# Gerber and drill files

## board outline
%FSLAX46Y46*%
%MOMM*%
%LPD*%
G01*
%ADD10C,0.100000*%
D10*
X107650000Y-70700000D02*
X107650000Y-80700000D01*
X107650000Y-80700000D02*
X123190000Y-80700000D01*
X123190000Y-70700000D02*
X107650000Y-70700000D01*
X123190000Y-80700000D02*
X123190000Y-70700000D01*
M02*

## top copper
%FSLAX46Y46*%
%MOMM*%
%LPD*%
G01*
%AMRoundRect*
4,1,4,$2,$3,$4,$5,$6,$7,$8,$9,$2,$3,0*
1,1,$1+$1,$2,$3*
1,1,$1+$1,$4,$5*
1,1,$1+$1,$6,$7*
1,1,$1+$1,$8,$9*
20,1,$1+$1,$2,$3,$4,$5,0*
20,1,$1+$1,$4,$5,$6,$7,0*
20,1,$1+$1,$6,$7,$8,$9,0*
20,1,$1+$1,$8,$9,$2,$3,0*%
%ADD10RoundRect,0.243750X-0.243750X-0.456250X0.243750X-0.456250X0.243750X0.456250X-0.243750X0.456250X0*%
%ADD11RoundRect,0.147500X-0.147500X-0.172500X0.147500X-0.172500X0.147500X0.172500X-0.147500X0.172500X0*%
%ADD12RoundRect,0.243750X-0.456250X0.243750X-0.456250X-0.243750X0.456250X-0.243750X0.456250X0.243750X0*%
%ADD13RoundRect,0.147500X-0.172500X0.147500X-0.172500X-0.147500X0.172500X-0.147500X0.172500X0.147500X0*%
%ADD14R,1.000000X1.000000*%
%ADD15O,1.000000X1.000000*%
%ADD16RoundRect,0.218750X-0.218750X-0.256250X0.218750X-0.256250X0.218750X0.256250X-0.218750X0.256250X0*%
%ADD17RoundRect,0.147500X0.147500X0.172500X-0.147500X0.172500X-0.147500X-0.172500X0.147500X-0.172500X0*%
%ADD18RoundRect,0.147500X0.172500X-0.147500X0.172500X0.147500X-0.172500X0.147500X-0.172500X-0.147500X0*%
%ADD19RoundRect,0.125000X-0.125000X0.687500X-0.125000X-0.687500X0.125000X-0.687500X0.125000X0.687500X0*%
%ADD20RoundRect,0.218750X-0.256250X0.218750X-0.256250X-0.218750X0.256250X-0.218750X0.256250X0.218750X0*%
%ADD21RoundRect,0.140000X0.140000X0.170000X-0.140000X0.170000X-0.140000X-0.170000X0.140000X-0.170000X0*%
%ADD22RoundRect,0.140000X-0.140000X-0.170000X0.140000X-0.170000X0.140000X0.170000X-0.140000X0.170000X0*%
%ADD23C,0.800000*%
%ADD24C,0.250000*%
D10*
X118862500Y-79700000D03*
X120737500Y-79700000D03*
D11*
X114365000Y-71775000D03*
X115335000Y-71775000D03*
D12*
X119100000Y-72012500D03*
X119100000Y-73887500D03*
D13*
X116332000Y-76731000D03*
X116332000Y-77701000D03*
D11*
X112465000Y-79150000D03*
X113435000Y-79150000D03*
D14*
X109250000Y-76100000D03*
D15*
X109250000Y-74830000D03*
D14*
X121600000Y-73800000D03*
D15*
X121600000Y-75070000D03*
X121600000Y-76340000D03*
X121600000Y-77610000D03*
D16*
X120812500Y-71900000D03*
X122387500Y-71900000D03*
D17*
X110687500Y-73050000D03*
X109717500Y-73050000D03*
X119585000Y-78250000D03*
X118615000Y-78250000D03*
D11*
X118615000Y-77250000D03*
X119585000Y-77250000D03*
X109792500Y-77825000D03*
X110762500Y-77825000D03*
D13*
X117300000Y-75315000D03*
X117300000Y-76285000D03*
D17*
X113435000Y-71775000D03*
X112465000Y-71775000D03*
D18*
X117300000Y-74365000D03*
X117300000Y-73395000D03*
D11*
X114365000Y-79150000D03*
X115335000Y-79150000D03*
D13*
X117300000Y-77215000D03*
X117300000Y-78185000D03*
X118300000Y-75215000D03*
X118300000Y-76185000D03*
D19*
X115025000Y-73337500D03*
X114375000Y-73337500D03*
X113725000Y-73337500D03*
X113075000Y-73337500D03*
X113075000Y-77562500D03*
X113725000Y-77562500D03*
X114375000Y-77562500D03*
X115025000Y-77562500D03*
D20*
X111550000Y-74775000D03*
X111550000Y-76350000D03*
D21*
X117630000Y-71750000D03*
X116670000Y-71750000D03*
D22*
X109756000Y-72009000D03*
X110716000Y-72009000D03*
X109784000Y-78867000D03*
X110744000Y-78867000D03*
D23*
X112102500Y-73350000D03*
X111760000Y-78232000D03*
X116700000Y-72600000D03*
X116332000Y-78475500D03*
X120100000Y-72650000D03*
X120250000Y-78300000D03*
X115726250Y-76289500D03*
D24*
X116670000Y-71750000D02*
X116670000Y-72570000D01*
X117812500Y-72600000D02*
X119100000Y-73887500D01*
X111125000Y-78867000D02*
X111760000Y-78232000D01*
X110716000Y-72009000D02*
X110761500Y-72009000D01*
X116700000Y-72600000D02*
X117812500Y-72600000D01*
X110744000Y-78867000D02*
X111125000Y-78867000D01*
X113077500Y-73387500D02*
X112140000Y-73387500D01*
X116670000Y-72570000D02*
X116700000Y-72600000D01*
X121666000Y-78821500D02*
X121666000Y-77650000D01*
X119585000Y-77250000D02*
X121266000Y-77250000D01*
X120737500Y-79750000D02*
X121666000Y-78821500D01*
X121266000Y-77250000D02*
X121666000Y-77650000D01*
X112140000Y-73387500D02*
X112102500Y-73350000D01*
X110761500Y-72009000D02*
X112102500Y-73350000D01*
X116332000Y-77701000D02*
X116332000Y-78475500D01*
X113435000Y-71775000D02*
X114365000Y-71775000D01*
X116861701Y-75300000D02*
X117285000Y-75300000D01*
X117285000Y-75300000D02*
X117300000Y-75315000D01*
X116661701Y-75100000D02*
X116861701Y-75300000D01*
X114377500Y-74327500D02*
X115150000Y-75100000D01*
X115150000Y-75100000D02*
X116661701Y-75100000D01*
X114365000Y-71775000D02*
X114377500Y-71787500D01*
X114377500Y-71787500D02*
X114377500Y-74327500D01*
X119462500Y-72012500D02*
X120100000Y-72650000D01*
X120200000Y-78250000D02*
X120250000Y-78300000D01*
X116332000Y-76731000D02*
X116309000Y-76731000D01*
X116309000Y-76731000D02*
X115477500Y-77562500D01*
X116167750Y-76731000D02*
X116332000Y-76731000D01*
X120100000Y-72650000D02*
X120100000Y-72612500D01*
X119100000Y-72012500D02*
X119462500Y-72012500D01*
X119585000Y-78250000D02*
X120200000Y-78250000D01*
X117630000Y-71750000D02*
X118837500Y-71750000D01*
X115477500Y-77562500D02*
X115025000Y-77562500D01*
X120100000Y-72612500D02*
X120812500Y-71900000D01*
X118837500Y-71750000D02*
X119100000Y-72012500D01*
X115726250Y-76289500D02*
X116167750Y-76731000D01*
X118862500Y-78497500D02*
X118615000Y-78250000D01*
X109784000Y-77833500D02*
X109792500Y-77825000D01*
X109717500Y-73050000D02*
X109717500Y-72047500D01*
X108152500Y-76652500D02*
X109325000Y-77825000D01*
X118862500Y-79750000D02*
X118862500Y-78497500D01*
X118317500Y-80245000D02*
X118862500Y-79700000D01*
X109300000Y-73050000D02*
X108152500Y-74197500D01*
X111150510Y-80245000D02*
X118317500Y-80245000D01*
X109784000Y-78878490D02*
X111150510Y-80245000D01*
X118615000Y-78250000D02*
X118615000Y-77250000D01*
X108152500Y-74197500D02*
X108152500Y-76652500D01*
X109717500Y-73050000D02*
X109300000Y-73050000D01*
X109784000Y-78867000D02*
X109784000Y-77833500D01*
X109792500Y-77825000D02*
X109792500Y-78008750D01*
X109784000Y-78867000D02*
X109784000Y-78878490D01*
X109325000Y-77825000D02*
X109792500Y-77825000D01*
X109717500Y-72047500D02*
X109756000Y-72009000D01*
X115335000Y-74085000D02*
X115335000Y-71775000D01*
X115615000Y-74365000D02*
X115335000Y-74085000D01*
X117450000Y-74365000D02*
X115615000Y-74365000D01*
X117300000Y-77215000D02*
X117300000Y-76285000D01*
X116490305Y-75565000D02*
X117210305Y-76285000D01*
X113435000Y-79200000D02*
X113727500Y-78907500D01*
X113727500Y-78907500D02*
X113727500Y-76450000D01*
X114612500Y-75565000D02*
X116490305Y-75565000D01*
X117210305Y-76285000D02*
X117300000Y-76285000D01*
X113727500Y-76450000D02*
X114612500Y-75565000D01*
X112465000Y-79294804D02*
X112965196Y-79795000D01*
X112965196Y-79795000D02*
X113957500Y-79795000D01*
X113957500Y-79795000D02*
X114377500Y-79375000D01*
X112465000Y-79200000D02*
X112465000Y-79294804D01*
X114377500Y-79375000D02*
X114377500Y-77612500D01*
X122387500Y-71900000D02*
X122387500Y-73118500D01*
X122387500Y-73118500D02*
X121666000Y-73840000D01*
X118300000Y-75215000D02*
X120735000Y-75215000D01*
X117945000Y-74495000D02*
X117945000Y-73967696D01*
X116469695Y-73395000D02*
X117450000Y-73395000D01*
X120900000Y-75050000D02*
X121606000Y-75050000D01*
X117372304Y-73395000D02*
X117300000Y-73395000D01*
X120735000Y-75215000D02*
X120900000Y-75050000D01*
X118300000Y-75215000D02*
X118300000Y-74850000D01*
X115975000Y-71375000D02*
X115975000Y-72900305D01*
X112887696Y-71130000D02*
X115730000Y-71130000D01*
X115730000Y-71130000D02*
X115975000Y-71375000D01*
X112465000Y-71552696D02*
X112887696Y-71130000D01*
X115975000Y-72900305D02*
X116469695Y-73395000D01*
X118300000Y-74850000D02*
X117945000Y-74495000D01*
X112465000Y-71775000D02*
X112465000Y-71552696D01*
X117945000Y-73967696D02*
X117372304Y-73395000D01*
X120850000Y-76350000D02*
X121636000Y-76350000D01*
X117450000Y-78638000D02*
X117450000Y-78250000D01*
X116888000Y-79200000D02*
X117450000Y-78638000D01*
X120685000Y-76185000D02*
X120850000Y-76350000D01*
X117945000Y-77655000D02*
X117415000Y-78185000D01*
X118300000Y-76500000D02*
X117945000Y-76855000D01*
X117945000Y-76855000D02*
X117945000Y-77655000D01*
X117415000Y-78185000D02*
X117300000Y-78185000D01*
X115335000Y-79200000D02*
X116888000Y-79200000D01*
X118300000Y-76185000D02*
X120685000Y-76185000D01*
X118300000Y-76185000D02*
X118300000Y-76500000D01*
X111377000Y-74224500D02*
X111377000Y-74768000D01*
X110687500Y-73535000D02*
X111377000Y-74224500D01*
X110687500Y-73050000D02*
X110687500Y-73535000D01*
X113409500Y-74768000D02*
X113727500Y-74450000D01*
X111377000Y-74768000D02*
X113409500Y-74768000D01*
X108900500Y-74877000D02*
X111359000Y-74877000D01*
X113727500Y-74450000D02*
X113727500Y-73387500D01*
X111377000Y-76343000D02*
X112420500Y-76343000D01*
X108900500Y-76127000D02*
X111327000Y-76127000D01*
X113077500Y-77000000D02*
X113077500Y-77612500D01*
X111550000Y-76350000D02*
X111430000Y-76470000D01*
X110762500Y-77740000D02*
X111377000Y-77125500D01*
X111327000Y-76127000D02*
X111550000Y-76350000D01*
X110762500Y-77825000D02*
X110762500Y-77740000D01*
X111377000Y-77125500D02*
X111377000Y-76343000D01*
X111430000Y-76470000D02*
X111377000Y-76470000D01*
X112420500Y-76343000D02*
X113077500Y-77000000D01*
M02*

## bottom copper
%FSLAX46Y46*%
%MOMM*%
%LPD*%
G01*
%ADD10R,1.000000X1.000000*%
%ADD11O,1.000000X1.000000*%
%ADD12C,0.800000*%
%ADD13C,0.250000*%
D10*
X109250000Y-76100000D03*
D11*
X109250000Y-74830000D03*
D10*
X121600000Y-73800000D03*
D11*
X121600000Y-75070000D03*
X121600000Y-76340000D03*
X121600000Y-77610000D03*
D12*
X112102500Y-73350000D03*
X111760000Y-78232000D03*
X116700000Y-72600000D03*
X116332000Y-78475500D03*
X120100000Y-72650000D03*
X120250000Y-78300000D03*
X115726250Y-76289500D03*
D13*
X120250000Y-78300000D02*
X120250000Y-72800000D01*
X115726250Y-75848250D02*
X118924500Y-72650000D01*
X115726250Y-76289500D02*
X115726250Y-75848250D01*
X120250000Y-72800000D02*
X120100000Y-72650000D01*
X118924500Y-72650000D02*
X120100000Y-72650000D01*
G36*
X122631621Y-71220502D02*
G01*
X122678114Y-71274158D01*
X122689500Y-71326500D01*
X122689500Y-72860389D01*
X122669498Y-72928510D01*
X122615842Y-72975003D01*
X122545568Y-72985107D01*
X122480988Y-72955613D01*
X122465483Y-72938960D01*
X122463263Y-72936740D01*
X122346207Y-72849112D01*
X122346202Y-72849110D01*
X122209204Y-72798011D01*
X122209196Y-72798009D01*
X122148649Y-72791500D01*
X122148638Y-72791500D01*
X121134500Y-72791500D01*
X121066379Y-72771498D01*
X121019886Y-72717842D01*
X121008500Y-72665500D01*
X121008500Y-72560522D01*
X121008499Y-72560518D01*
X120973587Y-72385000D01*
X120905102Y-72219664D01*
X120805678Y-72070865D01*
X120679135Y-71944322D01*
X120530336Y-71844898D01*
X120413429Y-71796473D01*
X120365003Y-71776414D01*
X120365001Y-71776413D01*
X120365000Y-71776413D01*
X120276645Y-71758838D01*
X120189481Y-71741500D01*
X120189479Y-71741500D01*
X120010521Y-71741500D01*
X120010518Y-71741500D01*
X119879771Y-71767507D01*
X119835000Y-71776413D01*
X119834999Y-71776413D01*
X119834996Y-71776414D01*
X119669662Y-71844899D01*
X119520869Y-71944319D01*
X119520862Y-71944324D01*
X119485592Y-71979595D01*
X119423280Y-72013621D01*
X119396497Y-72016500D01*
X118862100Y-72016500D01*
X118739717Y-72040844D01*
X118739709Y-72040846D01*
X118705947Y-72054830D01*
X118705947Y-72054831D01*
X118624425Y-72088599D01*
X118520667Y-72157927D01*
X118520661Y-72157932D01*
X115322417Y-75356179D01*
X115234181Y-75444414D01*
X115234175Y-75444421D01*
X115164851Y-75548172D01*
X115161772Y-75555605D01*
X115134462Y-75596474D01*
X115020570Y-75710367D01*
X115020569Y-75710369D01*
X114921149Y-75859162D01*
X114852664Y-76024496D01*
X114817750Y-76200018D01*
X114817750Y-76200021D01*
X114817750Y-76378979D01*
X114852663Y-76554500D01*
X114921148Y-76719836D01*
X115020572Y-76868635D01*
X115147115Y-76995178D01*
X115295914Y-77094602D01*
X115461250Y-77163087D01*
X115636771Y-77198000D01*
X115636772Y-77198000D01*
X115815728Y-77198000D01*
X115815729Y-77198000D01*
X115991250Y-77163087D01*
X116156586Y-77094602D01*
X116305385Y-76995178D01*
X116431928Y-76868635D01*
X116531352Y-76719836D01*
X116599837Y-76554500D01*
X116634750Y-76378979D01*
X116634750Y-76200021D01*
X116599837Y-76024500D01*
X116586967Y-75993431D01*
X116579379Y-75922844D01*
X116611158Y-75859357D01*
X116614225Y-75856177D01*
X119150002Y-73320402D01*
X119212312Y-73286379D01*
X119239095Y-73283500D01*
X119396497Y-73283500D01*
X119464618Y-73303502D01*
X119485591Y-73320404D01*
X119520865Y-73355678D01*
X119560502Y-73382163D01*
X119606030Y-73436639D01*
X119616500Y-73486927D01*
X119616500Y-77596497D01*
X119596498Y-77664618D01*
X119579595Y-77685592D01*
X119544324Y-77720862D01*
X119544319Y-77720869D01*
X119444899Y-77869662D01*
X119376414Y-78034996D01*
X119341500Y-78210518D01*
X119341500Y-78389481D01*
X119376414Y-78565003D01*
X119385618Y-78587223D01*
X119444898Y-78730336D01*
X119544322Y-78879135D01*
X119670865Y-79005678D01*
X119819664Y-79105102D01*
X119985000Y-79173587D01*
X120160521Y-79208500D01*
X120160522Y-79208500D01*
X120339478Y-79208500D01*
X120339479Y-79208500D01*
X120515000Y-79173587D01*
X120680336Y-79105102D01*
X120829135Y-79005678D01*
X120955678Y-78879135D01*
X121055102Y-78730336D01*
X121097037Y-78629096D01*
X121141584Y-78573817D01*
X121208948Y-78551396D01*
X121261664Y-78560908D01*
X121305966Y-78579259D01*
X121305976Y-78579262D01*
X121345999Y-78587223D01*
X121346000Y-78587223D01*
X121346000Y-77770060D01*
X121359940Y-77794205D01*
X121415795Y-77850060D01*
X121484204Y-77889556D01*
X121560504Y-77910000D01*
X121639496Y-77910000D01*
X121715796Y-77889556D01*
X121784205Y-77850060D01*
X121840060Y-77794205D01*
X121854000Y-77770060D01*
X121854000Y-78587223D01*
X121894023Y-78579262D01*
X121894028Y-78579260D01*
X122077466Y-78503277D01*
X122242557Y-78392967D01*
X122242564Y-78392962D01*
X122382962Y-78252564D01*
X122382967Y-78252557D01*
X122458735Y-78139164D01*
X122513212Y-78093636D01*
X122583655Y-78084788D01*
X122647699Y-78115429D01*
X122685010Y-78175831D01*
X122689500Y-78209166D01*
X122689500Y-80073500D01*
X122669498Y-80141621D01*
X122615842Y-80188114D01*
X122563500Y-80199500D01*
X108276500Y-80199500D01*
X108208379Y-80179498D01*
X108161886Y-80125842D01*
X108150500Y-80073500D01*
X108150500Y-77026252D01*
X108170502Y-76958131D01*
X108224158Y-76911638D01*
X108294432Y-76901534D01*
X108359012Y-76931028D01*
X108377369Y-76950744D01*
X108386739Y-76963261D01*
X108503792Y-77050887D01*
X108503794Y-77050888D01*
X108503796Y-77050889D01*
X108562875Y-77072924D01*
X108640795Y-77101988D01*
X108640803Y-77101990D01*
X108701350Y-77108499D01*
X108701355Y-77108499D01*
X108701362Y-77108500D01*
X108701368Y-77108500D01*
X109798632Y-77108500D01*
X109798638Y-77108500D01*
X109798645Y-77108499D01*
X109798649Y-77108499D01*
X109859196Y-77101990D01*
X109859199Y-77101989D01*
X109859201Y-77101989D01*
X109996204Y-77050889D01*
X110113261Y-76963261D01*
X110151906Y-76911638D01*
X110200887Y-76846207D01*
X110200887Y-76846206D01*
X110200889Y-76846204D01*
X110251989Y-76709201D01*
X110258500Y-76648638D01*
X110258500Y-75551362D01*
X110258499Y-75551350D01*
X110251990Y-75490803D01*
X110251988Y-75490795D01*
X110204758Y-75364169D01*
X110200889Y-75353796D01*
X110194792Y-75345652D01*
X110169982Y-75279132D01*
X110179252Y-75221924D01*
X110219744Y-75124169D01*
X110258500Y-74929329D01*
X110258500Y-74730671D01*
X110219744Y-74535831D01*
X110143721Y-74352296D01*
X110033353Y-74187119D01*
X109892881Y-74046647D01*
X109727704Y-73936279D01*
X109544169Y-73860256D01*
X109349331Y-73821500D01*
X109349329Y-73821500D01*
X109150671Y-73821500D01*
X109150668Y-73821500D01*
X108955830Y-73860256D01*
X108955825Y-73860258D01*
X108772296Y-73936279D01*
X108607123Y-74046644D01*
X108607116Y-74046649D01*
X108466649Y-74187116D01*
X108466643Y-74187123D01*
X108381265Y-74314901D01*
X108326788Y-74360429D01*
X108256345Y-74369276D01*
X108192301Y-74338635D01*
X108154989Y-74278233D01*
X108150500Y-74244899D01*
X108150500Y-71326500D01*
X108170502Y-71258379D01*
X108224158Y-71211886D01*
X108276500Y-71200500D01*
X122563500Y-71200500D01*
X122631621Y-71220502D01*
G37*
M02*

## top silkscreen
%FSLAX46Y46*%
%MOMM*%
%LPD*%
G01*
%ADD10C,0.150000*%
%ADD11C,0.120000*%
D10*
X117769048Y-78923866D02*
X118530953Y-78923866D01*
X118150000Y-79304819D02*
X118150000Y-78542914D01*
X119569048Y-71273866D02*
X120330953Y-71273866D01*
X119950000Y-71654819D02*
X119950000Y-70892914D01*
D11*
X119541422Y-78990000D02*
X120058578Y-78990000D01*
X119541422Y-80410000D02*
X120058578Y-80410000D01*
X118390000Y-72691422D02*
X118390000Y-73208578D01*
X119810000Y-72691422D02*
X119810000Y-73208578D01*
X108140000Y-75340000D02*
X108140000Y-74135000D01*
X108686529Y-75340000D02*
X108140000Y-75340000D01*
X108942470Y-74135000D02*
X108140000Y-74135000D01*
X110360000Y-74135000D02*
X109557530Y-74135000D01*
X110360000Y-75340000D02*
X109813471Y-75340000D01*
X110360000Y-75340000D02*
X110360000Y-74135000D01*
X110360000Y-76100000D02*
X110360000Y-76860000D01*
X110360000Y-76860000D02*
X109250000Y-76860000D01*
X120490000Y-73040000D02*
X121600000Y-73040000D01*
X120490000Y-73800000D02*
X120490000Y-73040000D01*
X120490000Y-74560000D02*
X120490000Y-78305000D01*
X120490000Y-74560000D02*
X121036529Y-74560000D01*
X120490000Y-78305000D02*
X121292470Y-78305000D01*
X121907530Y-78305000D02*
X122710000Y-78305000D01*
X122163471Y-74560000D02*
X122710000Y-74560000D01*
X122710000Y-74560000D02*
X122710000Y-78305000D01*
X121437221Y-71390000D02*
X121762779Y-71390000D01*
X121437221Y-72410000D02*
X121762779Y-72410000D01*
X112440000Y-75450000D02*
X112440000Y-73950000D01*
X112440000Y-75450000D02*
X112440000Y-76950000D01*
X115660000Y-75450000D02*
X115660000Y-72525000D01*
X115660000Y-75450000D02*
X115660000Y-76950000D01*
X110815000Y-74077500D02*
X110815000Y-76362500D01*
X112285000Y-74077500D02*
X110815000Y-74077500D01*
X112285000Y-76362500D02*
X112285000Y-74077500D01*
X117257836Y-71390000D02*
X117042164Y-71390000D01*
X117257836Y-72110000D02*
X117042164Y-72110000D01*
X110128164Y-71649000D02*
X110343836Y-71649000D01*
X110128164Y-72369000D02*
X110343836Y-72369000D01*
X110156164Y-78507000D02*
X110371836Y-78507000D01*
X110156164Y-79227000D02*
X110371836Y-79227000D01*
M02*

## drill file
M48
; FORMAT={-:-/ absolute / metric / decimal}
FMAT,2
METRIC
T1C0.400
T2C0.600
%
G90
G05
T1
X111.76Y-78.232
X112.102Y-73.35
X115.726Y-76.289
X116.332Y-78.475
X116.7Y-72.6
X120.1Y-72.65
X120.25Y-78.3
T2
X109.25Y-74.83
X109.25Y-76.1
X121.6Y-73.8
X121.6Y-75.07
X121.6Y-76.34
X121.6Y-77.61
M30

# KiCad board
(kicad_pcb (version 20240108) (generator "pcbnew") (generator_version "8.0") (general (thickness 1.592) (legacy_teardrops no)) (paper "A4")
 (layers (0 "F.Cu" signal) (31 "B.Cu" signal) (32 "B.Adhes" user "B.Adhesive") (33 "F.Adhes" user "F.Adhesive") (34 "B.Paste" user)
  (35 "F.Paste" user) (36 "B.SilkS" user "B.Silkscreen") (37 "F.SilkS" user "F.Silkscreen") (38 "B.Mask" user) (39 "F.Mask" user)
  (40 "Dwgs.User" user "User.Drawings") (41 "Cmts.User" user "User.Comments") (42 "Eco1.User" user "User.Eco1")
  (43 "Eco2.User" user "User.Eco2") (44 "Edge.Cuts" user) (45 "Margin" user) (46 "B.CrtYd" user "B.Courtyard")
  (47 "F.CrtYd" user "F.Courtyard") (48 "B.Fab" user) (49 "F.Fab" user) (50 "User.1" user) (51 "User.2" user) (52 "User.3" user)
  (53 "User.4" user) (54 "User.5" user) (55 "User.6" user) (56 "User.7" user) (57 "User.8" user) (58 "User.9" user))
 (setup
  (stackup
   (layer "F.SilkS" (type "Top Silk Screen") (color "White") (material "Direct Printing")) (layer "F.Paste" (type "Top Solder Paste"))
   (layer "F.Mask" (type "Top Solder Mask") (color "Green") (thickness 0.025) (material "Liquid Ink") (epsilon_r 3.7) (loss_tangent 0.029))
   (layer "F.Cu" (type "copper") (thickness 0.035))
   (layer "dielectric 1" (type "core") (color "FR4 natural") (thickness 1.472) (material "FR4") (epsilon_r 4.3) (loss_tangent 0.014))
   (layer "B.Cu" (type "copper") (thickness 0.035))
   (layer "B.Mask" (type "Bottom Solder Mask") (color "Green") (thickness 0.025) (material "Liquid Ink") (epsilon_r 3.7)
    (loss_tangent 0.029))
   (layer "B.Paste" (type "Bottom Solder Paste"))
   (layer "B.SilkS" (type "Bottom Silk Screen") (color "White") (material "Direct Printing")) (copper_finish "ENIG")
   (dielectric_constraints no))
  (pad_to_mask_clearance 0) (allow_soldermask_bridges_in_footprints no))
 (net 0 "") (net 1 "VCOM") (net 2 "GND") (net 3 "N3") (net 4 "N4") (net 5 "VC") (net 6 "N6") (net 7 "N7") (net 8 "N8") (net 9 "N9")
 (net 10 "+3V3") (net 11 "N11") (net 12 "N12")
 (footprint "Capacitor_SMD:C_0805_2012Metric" (layer "F.Cu") (at 119.8 79.7)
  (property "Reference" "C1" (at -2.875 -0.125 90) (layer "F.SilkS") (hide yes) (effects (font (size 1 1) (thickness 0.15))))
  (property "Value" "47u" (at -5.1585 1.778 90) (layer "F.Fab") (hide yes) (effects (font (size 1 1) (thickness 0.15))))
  (fp_line (start -0.258578 -0.71) (end 0.258578 -0.71) (stroke (width 0.12) (type solid)) (layer "F.SilkS"))
  (fp_line (start -0.258578 0.71) (end 0.258578 0.71) (stroke (width 0.12) (type solid)) (layer "F.SilkS"))
  (pad "1" smd roundrect (at -0.9375 0) (size 0.975 1.4) (layers "F.Cu" "F.Paste" "F.Mask") (roundrect_rratio 0.25) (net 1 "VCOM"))
  (pad "2" smd roundrect (at 0.9375 0) (size 0.975 1.4) (layers "F.Cu" "F.Paste" "F.Mask") (roundrect_rratio 0.25) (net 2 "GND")))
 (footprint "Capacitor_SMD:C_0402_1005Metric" (layer "F.Cu") (at 114.85 71.775)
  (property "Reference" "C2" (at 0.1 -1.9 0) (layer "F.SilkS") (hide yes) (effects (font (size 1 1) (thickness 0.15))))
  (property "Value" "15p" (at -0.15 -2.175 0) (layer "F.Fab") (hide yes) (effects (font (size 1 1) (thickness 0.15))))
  (pad "1" smd roundrect (at -0.485 0) (size 0.59 0.64) (layers "F.Cu" "F.Paste" "F.Mask") (roundrect_rratio 0.25) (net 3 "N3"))
  (pad "2" smd roundrect (at 0.485 0) (size 0.59 0.64) (layers "F.Cu" "F.Paste" "F.Mask") (roundrect_rratio 0.25) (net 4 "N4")))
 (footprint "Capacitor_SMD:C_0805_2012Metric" (layer "F.Cu") (at 119.1 72.95 -90)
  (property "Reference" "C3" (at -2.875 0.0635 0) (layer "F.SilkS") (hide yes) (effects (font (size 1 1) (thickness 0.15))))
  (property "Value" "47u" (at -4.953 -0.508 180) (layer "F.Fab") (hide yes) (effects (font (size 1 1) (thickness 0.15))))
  (fp_line (start -0.258578 0.71) (end 0.258578 0.71) (stroke (width 0.12) (type solid)) (layer "F.SilkS"))
  (fp_line (start -0.258578 -0.71) (end 0.258578 -0.71) (stroke (width 0.12) (type solid)) (layer "F.SilkS"))
  (pad "1" smd roundrect (at -0.9375 0 270) (size 0.975 1.4) (layers "F.Cu" "F.Paste" "F.Mask") (roundrect_rratio 0.25) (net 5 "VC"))
  (pad "2" smd roundrect (at 0.9375 0 270) (size 0.975 1.4) (layers "F.Cu" "F.Paste" "F.Mask") (roundrect_rratio 0.25) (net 2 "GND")))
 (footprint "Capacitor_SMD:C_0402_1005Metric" (layer "F.Cu") (at 116.332 77.216 -90)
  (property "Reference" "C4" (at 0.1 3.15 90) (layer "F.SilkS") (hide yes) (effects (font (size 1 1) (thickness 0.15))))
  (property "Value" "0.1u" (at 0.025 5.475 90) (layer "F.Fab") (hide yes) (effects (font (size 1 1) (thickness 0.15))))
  (pad "1" smd roundrect (at -0.485 0 270) (size 0.59 0.64) (layers "F.Cu" "F.Paste" "F.Mask") (roundrect_rratio 0.25) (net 5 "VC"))
  (pad "2" smd roundrect (at 0.485 0 270) (size 0.59 0.64) (layers "F.Cu" "F.Paste" "F.Mask") (roundrect_rratio 0.25) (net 2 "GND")))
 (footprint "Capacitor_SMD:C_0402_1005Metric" (layer "F.Cu") (at 112.95 79.15)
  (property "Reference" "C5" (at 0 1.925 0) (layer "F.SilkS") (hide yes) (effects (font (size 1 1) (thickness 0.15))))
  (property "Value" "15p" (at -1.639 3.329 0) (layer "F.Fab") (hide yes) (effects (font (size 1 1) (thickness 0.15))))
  (pad "1" smd roundrect (at -0.485 0) (size 0.59 0.64) (layers "F.Cu" "F.Paste" "F.Mask") (roundrect_rratio 0.25) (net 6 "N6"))
  (pad "2" smd roundrect (at 0.485 0) (size 0.59 0.64) (layers "F.Cu" "F.Paste" "F.Mask") (roundrect_rratio 0.25) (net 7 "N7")))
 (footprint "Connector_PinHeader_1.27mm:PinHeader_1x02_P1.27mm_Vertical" (layer "F.Cu") (at 109.25 76.1 180)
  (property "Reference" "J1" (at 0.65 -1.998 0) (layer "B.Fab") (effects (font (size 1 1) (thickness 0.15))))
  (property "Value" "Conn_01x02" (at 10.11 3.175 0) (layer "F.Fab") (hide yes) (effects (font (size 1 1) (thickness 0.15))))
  (fp_line (start 1.11 0.76) (end 1.11 1.965) (stroke (width 0.12) (type solid)) (layer "F.SilkS"))
  (fp_line (start 0.563471 0.76) (end 1.11 0.76) (stroke (width 0.12) (type solid)) (layer "F.SilkS"))
  (fp_line (start 0.30753 1.965) (end 1.11 1.965) (stroke (width 0.12) (type solid)) (layer "F.SilkS"))
  (fp_line (start -1.11 1.965) (end -0.30753 1.965) (stroke (width 0.12) (type solid)) (layer "F.SilkS"))
  (fp_line (start -1.11 0.76) (end -0.563471 0.76) (stroke (width 0.12) (type solid)) (layer "F.SilkS"))
  (fp_line (start -1.11 0.76) (end -1.11 1.965) (stroke (width 0.12) (type solid)) (layer "F.SilkS"))
  (fp_line (start -1.11 0) (end -1.11 -0.76) (stroke (width 0.12) (type solid)) (layer "F.SilkS"))
  (fp_line (start -1.11 -0.76) (end 0 -0.76) (stroke (width 0.12) (type solid)) (layer "F.SilkS"))
  (pad "1" thru_hole rect (at 0 0 180) (size 1 1) (drill 0.6) (layers "*.Cu" "*.Mask") (remove_unused_layers no) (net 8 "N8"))
  (pad "2" thru_hole oval (at 0 1.27 180) (size 1 1) (drill 0.6) (layers "*.Cu" "*.Mask") (remove_unused_layers no) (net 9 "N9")))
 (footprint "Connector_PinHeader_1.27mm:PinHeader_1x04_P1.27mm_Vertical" (layer "F.Cu") (at 121.6 73.8)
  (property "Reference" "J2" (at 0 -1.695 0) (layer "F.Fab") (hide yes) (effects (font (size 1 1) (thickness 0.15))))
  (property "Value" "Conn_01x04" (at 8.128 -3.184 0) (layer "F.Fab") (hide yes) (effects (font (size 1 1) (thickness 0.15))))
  (fp_line (start -1.11 -0.76) (end 0 -0.76) (stroke (width 0.12) (type solid)) (layer "F.SilkS"))
  (fp_line (start -1.11 0) (end -1.11 -0.76) (stroke (width 0.12) (type solid)) (layer "F.SilkS"))
  (fp_line (start -1.11 0.76) (end -1.11 4.505) (stroke (width 0.12) (type solid)) (layer "F.SilkS"))
  (fp_line (start -1.11 0.76) (end -0.563471 0.76) (stroke (width 0.12) (type solid)) (layer "F.SilkS"))
  (fp_line (start -1.11 4.505) (end -0.30753 4.505) (stroke (width 0.12) (type solid)) (layer "F.SilkS"))
  (fp_line (start 0.30753 4.505) (end 1.11 4.505) (stroke (width 0.12) (type solid)) (layer "F.SilkS"))
  (fp_line (start 0.563471 0.76) (end 1.11 0.76) (stroke (width 0.12) (type solid)) (layer "F.SilkS"))
  (fp_line (start 1.11 0.76) (end 1.11 4.505) (stroke (width 0.12) (type solid)) (layer "F.SilkS"))
  (pad "1" thru_hole rect (at 0 0) (size 1 1) (drill 0.6) (layers "*.Cu" "*.Mask") (remove_unused_layers no) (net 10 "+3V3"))
  (pad "2" thru_hole oval (at 0 1.27) (size 1 1) (drill 0.6) (layers "*.Cu" "*.Mask") (remove_unused_layers no) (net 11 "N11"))
  (pad "3" thru_hole oval (at 0 2.54) (size 1 1) (drill 0.6) (layers "*.Cu" "*.Mask") (remove_unused_layers no) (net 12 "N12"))
  (pad "4" thru_hole oval (at 0 3.81) (size 1 1) (drill 0.6) (layers "*.Cu" "*.Mask") (remove_unused_layers no) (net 2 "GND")))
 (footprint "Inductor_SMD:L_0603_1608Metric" (layer "F.Cu") (at 121.6 71.9)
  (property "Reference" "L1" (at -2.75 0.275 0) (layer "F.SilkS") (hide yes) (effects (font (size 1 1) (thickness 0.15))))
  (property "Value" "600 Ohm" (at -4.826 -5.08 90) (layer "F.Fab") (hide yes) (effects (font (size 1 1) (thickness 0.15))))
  (fp_line (start -0.162779 -0.51) (end 0.162779 -0.51) (stroke (width 0.12) (type solid)) (layer "F.SilkS"))
  (fp_line (start -0.162779 0.51) (end 0.162779 0.51) (stroke (width 0.12) (type solid)) (layer "F.SilkS"))
  (pad "1" smd roundrect (at -0.7875 0) (size 0.875 0.95) (layers "F.Cu" "F.Paste" "F.Mask") (roundrect_rratio 0.25) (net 5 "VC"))
  (pad "2" smd roundrect (at 0.7875 0) (size 0.875 0.95) (layers "F.Cu" "F.Paste" "F.Mask") (roundrect_rratio 0.25) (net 10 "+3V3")))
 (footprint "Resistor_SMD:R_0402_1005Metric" (layer "F.Cu") (at 110.2025 73.05 180)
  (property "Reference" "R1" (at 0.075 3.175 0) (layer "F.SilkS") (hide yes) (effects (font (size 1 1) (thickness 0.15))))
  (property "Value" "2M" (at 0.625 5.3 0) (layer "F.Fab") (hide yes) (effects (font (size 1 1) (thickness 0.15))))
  (pad "1" smd roundrect (at -0.485 0 180) (size 0.59 0.64) (layers "F.Cu" "F.Paste" "F.Mask") (roundrect_rratio 0.25) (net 9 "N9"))
  (pad "2" smd roundrect (at 0.485 0 180) (size 0.59 0.64) (layers "F.Cu" "F.Paste" "F.Mask") (roundrect_rratio 0.25) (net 1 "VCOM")))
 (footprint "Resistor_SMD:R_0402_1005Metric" (layer "F.Cu") (at 119.1 78.25 180)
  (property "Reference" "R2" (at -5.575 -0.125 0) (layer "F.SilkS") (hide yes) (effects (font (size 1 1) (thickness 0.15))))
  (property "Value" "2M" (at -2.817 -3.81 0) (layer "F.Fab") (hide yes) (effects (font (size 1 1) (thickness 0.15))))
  (pad "1" smd roundrect (at -0.485 0 180) (size 0.59 0.64) (layers "F.Cu" "F.Paste" "F.Mask") (roundrect_rratio 0.25) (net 5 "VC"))
  (pad "2" smd roundrect (at 0.485 0 180) (size 0.59 0.64) (layers "F.Cu" "F.Paste" "F.Mask") (roundrect_rratio 0.25) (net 1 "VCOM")))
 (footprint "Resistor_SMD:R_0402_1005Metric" (layer "F.Cu") (at 119.1 77.25)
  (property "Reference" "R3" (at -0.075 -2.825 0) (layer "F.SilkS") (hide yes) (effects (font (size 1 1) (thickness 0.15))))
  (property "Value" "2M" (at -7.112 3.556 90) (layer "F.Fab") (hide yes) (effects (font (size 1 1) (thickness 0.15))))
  (pad "1" smd roundrect (at -0.485 0) (size 0.59 0.64) (layers "F.Cu" "F.Paste" "F.Mask") (roundrect_rratio 0.25) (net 1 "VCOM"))
  (pad "2" smd roundrect (at 0.485 0) (size 0.59 0.64) (layers "F.Cu" "F.Paste" "F.Mask") (roundrect_rratio 0.25) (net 2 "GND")))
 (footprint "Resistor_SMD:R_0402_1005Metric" (layer "F.Cu") (at 110.2775 77.825)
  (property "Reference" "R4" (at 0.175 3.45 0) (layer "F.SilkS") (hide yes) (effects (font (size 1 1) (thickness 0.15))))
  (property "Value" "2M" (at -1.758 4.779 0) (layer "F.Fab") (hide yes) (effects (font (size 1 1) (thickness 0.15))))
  (pad "1" smd roundrect (at -0.485 0) (size 0.59 0.64) (layers "F.Cu" "F.Paste" "F.Mask") (roundrect_rratio 0.25) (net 1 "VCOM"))
  (pad "2" smd roundrect (at 0.485 0) (size 0.59 0.64) (layers "F.Cu" "F.Paste" "F.Mask") (roundrect_rratio 0.25) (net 8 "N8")))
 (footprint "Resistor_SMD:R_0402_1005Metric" (layer "F.Cu") (at 117.3 75.8 -90)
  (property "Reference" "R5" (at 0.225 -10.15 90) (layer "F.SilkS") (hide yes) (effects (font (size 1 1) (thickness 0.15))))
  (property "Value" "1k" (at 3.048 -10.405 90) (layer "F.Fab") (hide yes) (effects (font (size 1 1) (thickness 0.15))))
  (pad "1" smd roundrect (at -0.485 0 270) (size 0.59 0.64) (layers "F.Cu" "F.Paste" "F.Mask") (roundrect_rratio 0.25) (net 3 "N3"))
  (pad "2" smd roundrect (at 0.485 0 270) (size 0.59 0.64) (layers "F.Cu" "F.Paste" "F.Mask") (roundrect_rratio 0.25) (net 7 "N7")))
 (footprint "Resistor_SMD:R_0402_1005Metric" (layer "F.Cu") (at 112.95 71.775 180)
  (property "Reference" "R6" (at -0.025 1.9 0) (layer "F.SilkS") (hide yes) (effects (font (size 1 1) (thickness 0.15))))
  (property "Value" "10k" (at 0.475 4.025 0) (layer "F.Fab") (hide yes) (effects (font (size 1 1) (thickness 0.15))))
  (pad "1" smd roundrect (at -0.485 0 180) (size 0.59 0.64) (layers "F.Cu" "F.Paste" "F.Mask") (roundrect_rratio 0.25) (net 3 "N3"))
  (pad "2" smd roundrect (at 0.485 0 180) (size 0.59 0.64) (layers "F.Cu" "F.Paste" "F.Mask") (roundrect_rratio 0.25) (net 11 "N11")))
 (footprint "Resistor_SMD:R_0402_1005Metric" (layer "F.Cu") (at 117.3 73.88 90)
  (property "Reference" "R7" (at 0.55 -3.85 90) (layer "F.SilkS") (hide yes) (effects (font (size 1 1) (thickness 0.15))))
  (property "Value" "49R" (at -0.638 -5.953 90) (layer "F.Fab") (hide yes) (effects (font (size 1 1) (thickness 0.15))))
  (pad "1" smd roundrect (at -0.485 0 90) (size 0.59 0.64) (layers "F.Cu" "F.Paste" "F.Mask") (roundrect_rratio 0.25) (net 4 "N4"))
  (pad "2" smd roundrect (at 0.485 0 90) (size 0.59 0.64) (layers "F.Cu" "F.Paste" "F.Mask") (roundrect_rratio 0.25) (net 11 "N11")))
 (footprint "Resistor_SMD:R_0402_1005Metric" (layer "F.Cu") (at 114.85 79.15)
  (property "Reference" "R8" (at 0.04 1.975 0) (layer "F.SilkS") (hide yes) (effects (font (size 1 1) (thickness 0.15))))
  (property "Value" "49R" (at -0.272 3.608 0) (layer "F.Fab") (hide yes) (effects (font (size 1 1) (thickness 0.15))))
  (pad "1" smd roundrect (at -0.485 0) (size 0.59 0.64) (layers "F.Cu" "F.Paste" "F.Mask") (roundrect_rratio 0.25) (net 6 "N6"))
  (pad "2" smd roundrect (at 0.485 0) (size 0.59 0.64) (layers "F.Cu" "F.Paste" "F.Mask") (roundrect_rratio 0.25) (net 12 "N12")))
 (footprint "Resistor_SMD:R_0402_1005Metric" (layer "F.Cu") (at 117.3 77.7 -90)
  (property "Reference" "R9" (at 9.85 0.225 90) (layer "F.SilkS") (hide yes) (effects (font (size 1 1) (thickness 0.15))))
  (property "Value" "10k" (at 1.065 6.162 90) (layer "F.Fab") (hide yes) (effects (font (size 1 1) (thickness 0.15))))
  (pad "1" smd roundrect (at -0.485 0 270) (size 0.59 0.64) (layers "F.Cu" "F.Paste" "F.Mask") (roundrect_rratio 0.25) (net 7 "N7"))
  (pad "2" smd roundrect (at 0.485 0 270) (size 0.59 0.64) (layers "F.Cu" "F.Paste" "F.Mask") (roundrect_rratio 0.25) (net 12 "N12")))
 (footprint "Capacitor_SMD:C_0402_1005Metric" (layer "F.Cu") (at 118.3 75.7 -90)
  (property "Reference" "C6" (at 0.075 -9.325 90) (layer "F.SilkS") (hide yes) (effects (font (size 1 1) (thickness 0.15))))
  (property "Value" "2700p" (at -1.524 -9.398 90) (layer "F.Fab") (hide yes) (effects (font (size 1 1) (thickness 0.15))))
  (pad "1" smd roundrect (at -0.485 0 270) (size 0.59 0.64) (layers "F.Cu" "F.Paste" "F.Mask") (roundrect_rratio 0.25) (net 11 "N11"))
  (pad "2" smd roundrect (at 0.485 0 270) (size 0.59 0.64) (layers "F.Cu" "F.Paste" "F.Mask") (roundrect_rratio 0.25) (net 12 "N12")))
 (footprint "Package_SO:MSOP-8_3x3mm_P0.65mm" (layer "F.Cu") (at 114.05 75.45 -90)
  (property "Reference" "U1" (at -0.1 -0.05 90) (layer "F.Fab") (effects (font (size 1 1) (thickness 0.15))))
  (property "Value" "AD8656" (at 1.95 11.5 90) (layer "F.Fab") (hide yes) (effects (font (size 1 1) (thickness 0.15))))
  (fp_line (start 0 1.61) (end -1.5 1.61) (stroke (width 0.12) (type solid)) (layer "F.SilkS"))
  (fp_line (start 0 1.61) (end 1.5 1.61) (stroke (width 0.12) (type solid)) (layer "F.SilkS"))
  (fp_line (start 0 -1.61) (end -2.925 -1.61) (stroke (width 0.12) (type solid)) (layer "F.SilkS"))
  (fp_line (start 0 -1.61) (end 1.5 -1.61) (stroke (width 0.12) (type solid)) (layer "F.SilkS"))
  (pad "1" smd roundrect (at -2.1125 -0.975 270) (size 1.625 0.5) (layers "F.Cu" "F.Paste" "F.Mask") (roundrect_rratio 0.25) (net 4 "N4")
   (clearance 0.15))
  (pad "2" smd roundrect (at -2.1125 -0.325 270) (size 1.625 0.5) (layers "F.Cu" "F.Paste" "F.Mask") (roundrect_rratio 0.25) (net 3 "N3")
   (clearance 0.15))
  (pad "3" smd roundrect (at -2.1125 0.325 270) (size 1.625 0.5) (layers "F.Cu" "F.Paste" "F.Mask") (roundrect_rratio 0.25) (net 9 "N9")
   (clearance 0.15))
  (pad "4" smd roundrect (at -2.1125 0.975 270) (size 1.625 0.5) (layers "F.Cu" "F.Paste" "F.Mask") (roundrect_rratio 0.25) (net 2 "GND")
   (clearance 0.15))
  (pad "5" smd roundrect (at 2.1125 0.975 270) (size 1.625 0.5) (layers "F.Cu" "F.Paste" "F.Mask") (roundrect_rratio 0.25) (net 8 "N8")
   (clearance 0.15))
  (pad "6" smd roundrect (at 2.1125 0.325 270) (size 1.625 0.5) (layers "F.Cu" "F.Paste" "F.Mask") (roundrect_rratio 0.25) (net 7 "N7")
   (clearance 0.15))
  (pad "7" smd roundrect (at 2.1125 -0.325 270) (size 1.625 0.5) (layers "F.Cu" "F.Paste" "F.Mask") (roundrect_rratio 0.25) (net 6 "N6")
   (clearance 0.15))
  (pad "8" smd roundrect (at 2.1125 -0.975 270) (size 1.625 0.5) (layers "F.Cu" "F.Paste" "F.Mask") (roundrect_rratio 0.25) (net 5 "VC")
   (clearance 0.15)))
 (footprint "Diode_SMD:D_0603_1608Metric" (layer "F.Cu") (at 111.55 75.5625 -90)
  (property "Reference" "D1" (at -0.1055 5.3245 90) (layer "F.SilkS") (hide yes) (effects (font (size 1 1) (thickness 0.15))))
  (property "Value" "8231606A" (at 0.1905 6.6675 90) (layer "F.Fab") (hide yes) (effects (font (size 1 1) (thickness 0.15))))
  (fp_line (start -1.485 0.735) (end 0.8 0.735) (stroke (width 0.12) (type solid)) (layer "F.SilkS"))
  (fp_line (start -1.485 -0.735) (end -1.485 0.735) (stroke (width 0.12) (type solid)) (layer "F.SilkS"))
  (fp_line (start 0.8 -0.735) (end -1.485 -0.735) (stroke (width 0.12) (type solid)) (layer "F.SilkS"))
  (pad "1" smd roundrect (at -0.7875 0 270) (size 0.875 0.95) (layers "F.Cu" "F.Paste" "F.Mask") (roundrect_rratio 0.25) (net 9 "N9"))
  (pad "2" smd roundrect (at 0.7875 0 270) (size 0.875 0.95) (layers "F.Cu" "F.Paste" "F.Mask") (roundrect_rratio 0.25) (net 8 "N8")))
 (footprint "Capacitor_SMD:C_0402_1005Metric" (layer "F.Cu") (at 117.15 71.75 180)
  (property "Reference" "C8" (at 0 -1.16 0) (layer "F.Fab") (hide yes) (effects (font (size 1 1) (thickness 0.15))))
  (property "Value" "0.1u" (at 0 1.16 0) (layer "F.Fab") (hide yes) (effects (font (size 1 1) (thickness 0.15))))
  (fp_line (start -0.107836 0.36) (end 0.107836 0.36) (stroke (width 0.12) (type solid)) (layer "F.SilkS"))
  (fp_line (start -0.107836 -0.36) (end 0.107836 -0.36) (stroke (width 0.12) (type solid)) (layer "F.SilkS"))
  (pad "1" smd roundrect (at -0.48 0 180) (size 0.56 0.62) (layers "F.Cu" "F.Paste" "F.Mask") (roundrect_rratio 0.25) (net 5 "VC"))
  (pad "2" smd roundrect (at 0.48 0 180) (size 0.56 0.62) (layers "F.Cu" "F.Paste" "F.Mask") (roundrect_rratio 0.25) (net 2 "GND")))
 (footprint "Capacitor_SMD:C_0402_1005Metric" (layer "F.Cu") (at 110.236 72.009)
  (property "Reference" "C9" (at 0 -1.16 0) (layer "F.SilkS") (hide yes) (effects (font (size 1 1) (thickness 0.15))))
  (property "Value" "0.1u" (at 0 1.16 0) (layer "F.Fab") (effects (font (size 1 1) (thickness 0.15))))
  (fp_line (start -0.107836 -0.36) (end 0.107836 -0.36) (stroke (width 0.12) (type solid)) (layer "F.SilkS"))
  (fp_line (start -0.107836 0.36) (end 0.107836 0.36) (stroke (width 0.12) (type solid)) (layer "F.SilkS"))
  (pad "1" smd roundrect (at -0.48 0) (size 0.56 0.62) (layers "F.Cu" "F.Paste" "F.Mask") (roundrect_rratio 0.25) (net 1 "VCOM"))
  (pad "2" smd roundrect (at 0.48 0) (size 0.56 0.62) (layers "F.Cu" "F.Paste" "F.Mask") (roundrect_rratio 0.25) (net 2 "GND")))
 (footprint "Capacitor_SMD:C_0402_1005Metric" (layer "F.Cu") (at 110.264 78.867)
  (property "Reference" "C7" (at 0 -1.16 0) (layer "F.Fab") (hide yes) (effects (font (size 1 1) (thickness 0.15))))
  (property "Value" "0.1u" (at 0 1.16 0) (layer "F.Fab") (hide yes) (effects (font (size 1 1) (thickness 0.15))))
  (fp_line (start -0.107836 -0.36) (end 0.107836 -0.36) (stroke (width 0.12) (type solid)) (layer "F.SilkS"))
  (fp_line (start -0.107836 0.36) (end 0.107836 0.36) (stroke (width 0.12) (type solid)) (layer "F.SilkS"))
  (pad "1" smd roundrect (at -0.48 0) (size 0.56 0.62) (layers "F.Cu" "F.Paste" "F.Mask") (roundrect_rratio 0.25) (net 1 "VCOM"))
  (pad "2" smd roundrect (at 0.48 0) (size 0.56 0.62) (layers "F.Cu" "F.Paste" "F.Mask") (roundrect_rratio 0.25) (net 2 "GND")))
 (gr_line (start 107.65 70.7) (end 107.65 80.7) (stroke (width 0.1) (type solid)) (layer "Edge.Cuts"))
 (gr_line (start 107.65 80.7) (end 123.19 80.7) (stroke (width 0.1) (type solid)) (layer "Edge.Cuts"))
 (gr_line (start 123.19 70.7) (end 107.65 70.7) (stroke (width 0.1) (type solid)) (layer "Edge.Cuts"))
 (gr_line (start 123.19 80.7) (end 123.19 70.7) (stroke (width 0.1) (type solid)) (layer "Edge.Cuts"))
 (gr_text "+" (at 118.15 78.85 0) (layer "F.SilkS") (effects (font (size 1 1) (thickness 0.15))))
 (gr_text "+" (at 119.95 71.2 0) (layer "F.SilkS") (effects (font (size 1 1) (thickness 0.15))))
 (segment (start 116.67 71.75) (end 116.67 72.57) (width 0.25) (layer "F.Cu") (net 2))
 (segment (start 117.8125 72.6) (end 119.1 73.8875) (width 0.25) (layer "F.Cu") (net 2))
 (segment (start 111.125 78.867) (end 111.76 78.232) (width 0.25) (layer "F.Cu") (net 2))
 (segment (start 110.716 72.009) (end 110.7615 72.009) (width 0.25) (layer "F.Cu") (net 2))
 (segment (start 116.7 72.6) (end 117.8125 72.6) (width 0.25) (layer "F.Cu") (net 2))
 (segment (start 110.744 78.867) (end 111.125 78.867) (width 0.25) (layer "F.Cu") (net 2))
 (segment (start 113.0775 73.3875) (end 112.14 73.3875) (width 0.25) (layer "F.Cu") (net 2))
 (segment (start 116.67 72.57) (end 116.7 72.6) (width 0.25) (layer "F.Cu") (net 2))
 (segment (start 121.666 78.8215) (end 121.666 77.65) (width 0.25) (layer "F.Cu") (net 2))
 (segment (start 119.585 77.25) (end 121.266 77.25) (width 0.25) (layer "F.Cu") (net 2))
 (segment (start 120.7375 79.75) (end 121.666 78.8215) (width 0.25) (layer "F.Cu") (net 2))
 (segment (start 121.266 77.25) (end 121.666 77.65) (width 0.25) (layer "F.Cu") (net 2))
 (segment (start 112.14 73.3875) (end 112.1025 73.35) (width 0.25) (layer "F.Cu") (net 2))
 (segment (start 110.7615 72.009) (end 112.1025 73.35) (width 0.25) (layer "F.Cu") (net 2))
 (segment (start 116.332 77.701) (end 116.332 78.4755) (width 0.25) (layer "F.Cu") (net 2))
 (via (at 112.1025 73.35) (size 0.8) (drill 0.4) (layers "F.Cu" "B.Cu") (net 2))
 (via (at 111.76 78.232) (size 0.8) (drill 0.4) (layers "F.Cu" "B.Cu") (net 2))
 (via (at 116.7 72.6) (size 0.8) (drill 0.4) (layers "F.Cu" "B.Cu") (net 2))
 (via (at 116.332 78.4755) (size 0.8) (drill 0.4) (layers "F.Cu" "B.Cu") (free yes) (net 2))
 (segment (start 113.435 71.775) (end 114.365 71.775) (width 0.25) (layer "F.Cu") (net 3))
 (segment (start 116.861701 75.3) (end 117.285 75.3) (width 0.25) (layer "F.Cu") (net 3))
 (segment (start 117.285 75.3) (end 117.3 75.315) (width 0.25) (layer "F.Cu") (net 3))
 (segment (start 116.661701 75.1) (end 116.861701 75.3) (width 0.25) (layer "F.Cu") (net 3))
 (segment (start 114.3775 74.3275) (end 115.15 75.1) (width 0.25) (layer "F.Cu") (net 3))
 (segment (start 115.15 75.1) (end 116.661701 75.1) (width 0.25) (layer "F.Cu") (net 3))
 (segment (start 114.365 71.775) (end 114.3775 71.7875) (width 0.25) (layer "F.Cu") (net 3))
 (segment (start 114.3775 71.7875) (end 114.3775 74.3275) (width 0.25) (layer "F.Cu") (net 3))
 (segment (start 119.4625 72.0125) (end 120.1 72.65) (width 0.25) (layer "F.Cu") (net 5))
 (segment (start 120.2 78.25) (end 120.25 78.3) (width 0.25) (layer "F.Cu") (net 5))
 (segment (start 116.332 76.731) (end 116.309 76.731) (width 0.25) (layer "F.Cu") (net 5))
 (segment (start 116.309 76.731) (end 115.4775 77.5625) (width 0.25) (layer "F.Cu") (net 5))
 (segment (start 116.16775 76.731) (end 116.332 76.731) (width 0.25) (layer "F.Cu") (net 5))
 (segment (start 120.1 72.65) (end 120.1 72.6125) (width 0.25) (layer "F.Cu") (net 5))
 (segment (start 119.1 72.0125) (end 119.4625 72.0125) (width 0.25) (layer "F.Cu") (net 5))
 (segment (start 119.585 78.25) (end 120.2 78.25) (width 0.25) (layer "F.Cu") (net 5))
 (segment (start 117.63 71.75) (end 118.8375 71.75) (width 0.25) (layer "F.Cu") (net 5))
 (segment (start 115.4775 77.5625) (end 115.025 77.5625) (width 0.25) (layer "F.Cu") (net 5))
 (segment (start 120.1 72.6125) (end 120.8125 71.9) (width 0.25) (layer "F.Cu") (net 5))
 (segment (start 118.8375 71.75) (end 119.1 72.0125) (width 0.25) (layer "F.Cu") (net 5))
 (segment (start 115.72625 76.2895) (end 116.16775 76.731) (width 0.25) (layer "F.Cu") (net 5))
 (via (at 120.1 72.65) (size 0.8) (drill 0.4) (layers "F.Cu" "B.Cu") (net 5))
 (via (at 120.25 78.3) (size 0.8) (drill 0.4) (layers "F.Cu" "B.Cu") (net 5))
 (via (at 115.72625 76.2895) (size 0.8) (drill 0.4) (layers "F.Cu" "B.Cu") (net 5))
 (segment (start 120.25 78.3) (end 120.25 72.8) (width 0.25) (layer "B.Cu") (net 5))
 (segment (start 115.72625 75.84825) (end 118.9245 72.65) (width 0.25) (layer "B.Cu") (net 5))
 (segment (start 115.72625 76.2895) (end 115.72625 75.84825) (width 0.25) (layer "B.Cu") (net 5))
 (segment (start 120.25 72.8) (end 120.1 72.65) (width 0.25) (layer "B.Cu") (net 5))
 (segment (start 118.9245 72.65) (end 120.1 72.65) (width 0.25) (layer "B.Cu") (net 5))
 (segment (start 118.8625 78.4975) (end 118.615 78.25) (width 0.25) (layer "F.Cu") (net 1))
 (segment (start 109.784 77.8335) (end 109.7925 77.825) (width 0.25) (layer "F.Cu") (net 1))
 (segment (start 109.7175 73.05) (end 109.7175 72.0475) (width 0.25) (layer "F.Cu") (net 1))
 (segment (start 108.1525 76.6525) (end 109.325 77.825) (width 0.25) (layer "F.Cu") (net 1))
 (segment (start 118.8625 79.75) (end 118.8625 78.4975) (width 0.25) (layer "F.Cu") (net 1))
 (segment (start 118.3175 80.245) (end 118.8625 79.7) (width 0.25) (layer "F.Cu") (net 1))
 (segment (start 109.3 73.05) (end 108.1525 74.1975) (width 0.25) (layer "F.Cu") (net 1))
 (segment (start 111.15051 80.245) (end 118.3175 80.245) (width 0.25) (layer "F.Cu") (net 1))
 (segment (start 109.784 78.87849) (end 111.15051 80.245) (width 0.25) (layer "F.Cu") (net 1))
 (segment (start 118.615 78.25) (end 118.615 77.25) (width 0.25) (layer "F.Cu") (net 1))
 (segment (start 108.1525 74.1975) (end 108.1525 76.6525) (width 0.25) (layer "F.Cu") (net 1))
 (segment (start 109.7175 73.05) (end 109.3 73.05) (width 0.25) (layer "F.Cu") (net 1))
 (segment (start 109.784 78.867) (end 109.784 77.8335) (width 0.25) (layer "F.Cu") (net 1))
 (segment (start 109.7925 77.825) (end 109.7925 78.00875) (width 0.25) (layer "F.Cu") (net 1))
 (segment (start 109.784 78.867) (end 109.784 78.87849) (width 0.25) (layer "F.Cu") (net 1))
 (segment (start 109.325 77.825) (end 109.7925 77.825) (width 0.25) (layer "F.Cu") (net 1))
 (segment (start 109.7175 72.0475) (end 109.756 72.009) (width 0.25) (layer "F.Cu") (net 1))
 (segment (start 115.335 74.085) (end 115.335 71.775) (width 0.25) (layer "F.Cu") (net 4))
 (segment (start 115.615 74.365) (end 115.335 74.085) (width 0.25) (layer "F.Cu") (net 4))
 (segment (start 117.45 74.365) (end 115.615 74.365) (width 0.25) (layer "F.Cu") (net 4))
 (segment (start 117.3 77.215) (end 117.3 76.285) (width 0.25) (layer "F.Cu") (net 7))
 (segment (start 116.490305 75.565) (end 117.210305 76.285) (width 0.25) (layer "F.Cu") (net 7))
 (segment (start 113.435 79.2) (end 113.7275 78.9075) (width 0.25) (layer "F.Cu") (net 7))
 (segment (start 113.7275 78.9075) (end 113.7275 76.45) (width 0.25) (layer "F.Cu") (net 7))
 (segment (start 114.6125 75.565) (end 116.490305 75.565) (width 0.25) (layer "F.Cu") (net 7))
 (segment (start 117.210305 76.285) (end 117.3 76.285) (width 0.25) (layer "F.Cu") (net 7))
 (segment (start 113.7275 76.45) (end 114.6125 75.565) (width 0.25) (layer "F.Cu") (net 7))
 (segment (start 112.465 79.294804) (end 112.965196 79.795) (width 0.25) (layer "F.Cu") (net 6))
 (segment (start 112.965196 79.795) (end 113.9575 79.795) (width 0.25) (layer "F.Cu") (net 6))
 (segment (start 113.9575 79.795) (end 114.3775 79.375) (width 0.25) (layer "F.Cu") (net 6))
 (segment (start 112.465 79.2) (end 112.465 79.294804) (width 0.25) (layer "F.Cu") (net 6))
 (segment (start 114.3775 79.375) (end 114.3775 77.6125) (width 0.25) (layer "F.Cu") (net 6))
 (segment (start 122.3875 71.9) (end 122.3875 73.1185) (width 0.25) (layer "F.Cu") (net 10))
 (segment (start 122.3875 73.1185) (end 121.666 73.84) (width 0.25) (layer "F.Cu") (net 10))
 (segment (start 118.3 75.215) (end 120.735 75.215) (width 0.25) (layer "F.Cu") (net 11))
 (segment (start 117.945 74.495) (end 117.945 73.967696) (width 0.25) (layer "F.Cu") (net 11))
 (segment (start 116.469695 73.395) (end 117.45 73.395) (width 0.25) (layer "F.Cu") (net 11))
 (segment (start 120.9 75.05) (end 121.606 75.05) (width 0.25) (layer "F.Cu") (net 11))
 (segment (start 117.372304 73.395) (end 117.3 73.395) (width 0.25) (layer "F.Cu") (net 11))
 (segment (start 120.735 75.215) (end 120.9 75.05) (width 0.25) (layer "F.Cu") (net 11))
 (segment (start 118.3 75.215) (end 118.3 74.85) (width 0.25) (layer "F.Cu") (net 11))
 (segment (start 115.975 71.375) (end 115.975 72.900305) (width 0.25) (layer "F.Cu") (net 11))
 (segment (start 112.887696 71.13) (end 115.73 71.13) (width 0.25) (layer "F.Cu") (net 11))
 (segment (start 115.73 71.13) (end 115.975 71.375) (width 0.25) (layer "F.Cu") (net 11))
 (segment (start 112.465 71.552696) (end 112.887696 71.13) (width 0.25) (layer "F.Cu") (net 11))
 (segment (start 115.975 72.900305) (end 116.469695 73.395) (width 0.25) (layer "F.Cu") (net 11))
 (segment (start 118.3 74.85) (end 117.945 74.495) (width 0.25) (layer "F.Cu") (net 11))
 (segment (start 112.465 71.775) (end 112.465 71.552696) (width 0.25) (layer "F.Cu") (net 11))
 (segment (start 117.945 73.967696) (end 117.372304 73.395) (width 0.25) (layer "F.Cu") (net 11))
 (segment (start 120.85 76.35) (end 121.636 76.35) (width 0.25) (layer "F.Cu") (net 12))
 (segment (start 117.45 78.638) (end 117.45 78.25) (width 0.25) (layer "F.Cu") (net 12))
 (segment (start 116.888 79.2) (end 117.45 78.638) (width 0.25) (layer "F.Cu") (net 12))
 (segment (start 120.685 76.185) (end 120.85 76.35) (width 0.25) (layer "F.Cu") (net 12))
 (segment (start 117.945 77.655) (end 117.415 78.185) (width 0.25) (layer "F.Cu") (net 12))
 (segment (start 118.3 76.5) (end 117.945 76.855) (width 0.25) (layer "F.Cu") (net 12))
 (segment (start 117.945 76.855) (end 117.945 77.655) (width 0.25) (layer "F.Cu") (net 12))
 (segment (start 117.415 78.185) (end 117.3 78.185) (width 0.25) (layer "F.Cu") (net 12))
 (segment (start 115.335 79.2) (end 116.888 79.2) (width 0.25) (layer "F.Cu") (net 12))
 (segment (start 118.3 76.185) (end 120.685 76.185) (width 0.25) (layer "F.Cu") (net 12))
 (segment (start 118.3 76.185) (end 118.3 76.5) (width 0.25) (layer "F.Cu") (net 12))
 (segment (start 111.377 74.2245) (end 111.377 74.768) (width 0.25) (layer "F.Cu") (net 9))
 (segment (start 110.6875 73.535) (end 111.377 74.2245) (width 0.25) (layer "F.Cu") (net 9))
 (segment (start 110.6875 73.05) (end 110.6875 73.535) (width 0.25) (layer "F.Cu") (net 9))
 (segment (start 113.4095 74.768) (end 113.7275 74.45) (width 0.25) (layer "F.Cu") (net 9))
 (segment (start 111.377 74.768) (end 113.4095 74.768) (width 0.25) (layer "F.Cu") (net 9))
 (segment (start 108.9005 74.877) (end 111.359 74.877) (width 0.25) (layer "F.Cu") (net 9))
 (segment (start 113.7275 74.45) (end 113.7275 73.3875) (width 0.25) (layer "F.Cu") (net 9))
 (segment (start 111.377 76.343) (end 112.4205 76.343) (width 0.25) (layer "F.Cu") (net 8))
 (segment (start 108.9005 76.127) (end 111.327 76.127) (width 0.25) (layer "F.Cu") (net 8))
 (segment (start 113.0775 77) (end 113.0775 77.6125) (width 0.25) (layer "F.Cu") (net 8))
 (segment (start 111.55 76.35) (end 111.43 76.47) (width 0.25) (layer "F.Cu") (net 8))
 (segment (start 110.7625 77.74) (end 111.377 77.1255) (width 0.25) (layer "F.Cu") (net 8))
 (segment (start 111.327 76.127) (end 111.55 76.35) (width 0.25) (layer "F.Cu") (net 8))
 (segment (start 110.7625 77.825) (end 110.7625 77.74) (width 0.25) (layer "F.Cu") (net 8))
 (segment (start 111.377 77.1255) (end 111.377 76.343) (width 0.25) (layer "F.Cu") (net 8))
 (segment (start 111.43 76.47) (end 111.377 76.47) (width 0.25) (layer "F.Cu") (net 8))
 (segment (start 112.4205 76.343) (end 113.0775 77) (width 0.25) (layer "F.Cu") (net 8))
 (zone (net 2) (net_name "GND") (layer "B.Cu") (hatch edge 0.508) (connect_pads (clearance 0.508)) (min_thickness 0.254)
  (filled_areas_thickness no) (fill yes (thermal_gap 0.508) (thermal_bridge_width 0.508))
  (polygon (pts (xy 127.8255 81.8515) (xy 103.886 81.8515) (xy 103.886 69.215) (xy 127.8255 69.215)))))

